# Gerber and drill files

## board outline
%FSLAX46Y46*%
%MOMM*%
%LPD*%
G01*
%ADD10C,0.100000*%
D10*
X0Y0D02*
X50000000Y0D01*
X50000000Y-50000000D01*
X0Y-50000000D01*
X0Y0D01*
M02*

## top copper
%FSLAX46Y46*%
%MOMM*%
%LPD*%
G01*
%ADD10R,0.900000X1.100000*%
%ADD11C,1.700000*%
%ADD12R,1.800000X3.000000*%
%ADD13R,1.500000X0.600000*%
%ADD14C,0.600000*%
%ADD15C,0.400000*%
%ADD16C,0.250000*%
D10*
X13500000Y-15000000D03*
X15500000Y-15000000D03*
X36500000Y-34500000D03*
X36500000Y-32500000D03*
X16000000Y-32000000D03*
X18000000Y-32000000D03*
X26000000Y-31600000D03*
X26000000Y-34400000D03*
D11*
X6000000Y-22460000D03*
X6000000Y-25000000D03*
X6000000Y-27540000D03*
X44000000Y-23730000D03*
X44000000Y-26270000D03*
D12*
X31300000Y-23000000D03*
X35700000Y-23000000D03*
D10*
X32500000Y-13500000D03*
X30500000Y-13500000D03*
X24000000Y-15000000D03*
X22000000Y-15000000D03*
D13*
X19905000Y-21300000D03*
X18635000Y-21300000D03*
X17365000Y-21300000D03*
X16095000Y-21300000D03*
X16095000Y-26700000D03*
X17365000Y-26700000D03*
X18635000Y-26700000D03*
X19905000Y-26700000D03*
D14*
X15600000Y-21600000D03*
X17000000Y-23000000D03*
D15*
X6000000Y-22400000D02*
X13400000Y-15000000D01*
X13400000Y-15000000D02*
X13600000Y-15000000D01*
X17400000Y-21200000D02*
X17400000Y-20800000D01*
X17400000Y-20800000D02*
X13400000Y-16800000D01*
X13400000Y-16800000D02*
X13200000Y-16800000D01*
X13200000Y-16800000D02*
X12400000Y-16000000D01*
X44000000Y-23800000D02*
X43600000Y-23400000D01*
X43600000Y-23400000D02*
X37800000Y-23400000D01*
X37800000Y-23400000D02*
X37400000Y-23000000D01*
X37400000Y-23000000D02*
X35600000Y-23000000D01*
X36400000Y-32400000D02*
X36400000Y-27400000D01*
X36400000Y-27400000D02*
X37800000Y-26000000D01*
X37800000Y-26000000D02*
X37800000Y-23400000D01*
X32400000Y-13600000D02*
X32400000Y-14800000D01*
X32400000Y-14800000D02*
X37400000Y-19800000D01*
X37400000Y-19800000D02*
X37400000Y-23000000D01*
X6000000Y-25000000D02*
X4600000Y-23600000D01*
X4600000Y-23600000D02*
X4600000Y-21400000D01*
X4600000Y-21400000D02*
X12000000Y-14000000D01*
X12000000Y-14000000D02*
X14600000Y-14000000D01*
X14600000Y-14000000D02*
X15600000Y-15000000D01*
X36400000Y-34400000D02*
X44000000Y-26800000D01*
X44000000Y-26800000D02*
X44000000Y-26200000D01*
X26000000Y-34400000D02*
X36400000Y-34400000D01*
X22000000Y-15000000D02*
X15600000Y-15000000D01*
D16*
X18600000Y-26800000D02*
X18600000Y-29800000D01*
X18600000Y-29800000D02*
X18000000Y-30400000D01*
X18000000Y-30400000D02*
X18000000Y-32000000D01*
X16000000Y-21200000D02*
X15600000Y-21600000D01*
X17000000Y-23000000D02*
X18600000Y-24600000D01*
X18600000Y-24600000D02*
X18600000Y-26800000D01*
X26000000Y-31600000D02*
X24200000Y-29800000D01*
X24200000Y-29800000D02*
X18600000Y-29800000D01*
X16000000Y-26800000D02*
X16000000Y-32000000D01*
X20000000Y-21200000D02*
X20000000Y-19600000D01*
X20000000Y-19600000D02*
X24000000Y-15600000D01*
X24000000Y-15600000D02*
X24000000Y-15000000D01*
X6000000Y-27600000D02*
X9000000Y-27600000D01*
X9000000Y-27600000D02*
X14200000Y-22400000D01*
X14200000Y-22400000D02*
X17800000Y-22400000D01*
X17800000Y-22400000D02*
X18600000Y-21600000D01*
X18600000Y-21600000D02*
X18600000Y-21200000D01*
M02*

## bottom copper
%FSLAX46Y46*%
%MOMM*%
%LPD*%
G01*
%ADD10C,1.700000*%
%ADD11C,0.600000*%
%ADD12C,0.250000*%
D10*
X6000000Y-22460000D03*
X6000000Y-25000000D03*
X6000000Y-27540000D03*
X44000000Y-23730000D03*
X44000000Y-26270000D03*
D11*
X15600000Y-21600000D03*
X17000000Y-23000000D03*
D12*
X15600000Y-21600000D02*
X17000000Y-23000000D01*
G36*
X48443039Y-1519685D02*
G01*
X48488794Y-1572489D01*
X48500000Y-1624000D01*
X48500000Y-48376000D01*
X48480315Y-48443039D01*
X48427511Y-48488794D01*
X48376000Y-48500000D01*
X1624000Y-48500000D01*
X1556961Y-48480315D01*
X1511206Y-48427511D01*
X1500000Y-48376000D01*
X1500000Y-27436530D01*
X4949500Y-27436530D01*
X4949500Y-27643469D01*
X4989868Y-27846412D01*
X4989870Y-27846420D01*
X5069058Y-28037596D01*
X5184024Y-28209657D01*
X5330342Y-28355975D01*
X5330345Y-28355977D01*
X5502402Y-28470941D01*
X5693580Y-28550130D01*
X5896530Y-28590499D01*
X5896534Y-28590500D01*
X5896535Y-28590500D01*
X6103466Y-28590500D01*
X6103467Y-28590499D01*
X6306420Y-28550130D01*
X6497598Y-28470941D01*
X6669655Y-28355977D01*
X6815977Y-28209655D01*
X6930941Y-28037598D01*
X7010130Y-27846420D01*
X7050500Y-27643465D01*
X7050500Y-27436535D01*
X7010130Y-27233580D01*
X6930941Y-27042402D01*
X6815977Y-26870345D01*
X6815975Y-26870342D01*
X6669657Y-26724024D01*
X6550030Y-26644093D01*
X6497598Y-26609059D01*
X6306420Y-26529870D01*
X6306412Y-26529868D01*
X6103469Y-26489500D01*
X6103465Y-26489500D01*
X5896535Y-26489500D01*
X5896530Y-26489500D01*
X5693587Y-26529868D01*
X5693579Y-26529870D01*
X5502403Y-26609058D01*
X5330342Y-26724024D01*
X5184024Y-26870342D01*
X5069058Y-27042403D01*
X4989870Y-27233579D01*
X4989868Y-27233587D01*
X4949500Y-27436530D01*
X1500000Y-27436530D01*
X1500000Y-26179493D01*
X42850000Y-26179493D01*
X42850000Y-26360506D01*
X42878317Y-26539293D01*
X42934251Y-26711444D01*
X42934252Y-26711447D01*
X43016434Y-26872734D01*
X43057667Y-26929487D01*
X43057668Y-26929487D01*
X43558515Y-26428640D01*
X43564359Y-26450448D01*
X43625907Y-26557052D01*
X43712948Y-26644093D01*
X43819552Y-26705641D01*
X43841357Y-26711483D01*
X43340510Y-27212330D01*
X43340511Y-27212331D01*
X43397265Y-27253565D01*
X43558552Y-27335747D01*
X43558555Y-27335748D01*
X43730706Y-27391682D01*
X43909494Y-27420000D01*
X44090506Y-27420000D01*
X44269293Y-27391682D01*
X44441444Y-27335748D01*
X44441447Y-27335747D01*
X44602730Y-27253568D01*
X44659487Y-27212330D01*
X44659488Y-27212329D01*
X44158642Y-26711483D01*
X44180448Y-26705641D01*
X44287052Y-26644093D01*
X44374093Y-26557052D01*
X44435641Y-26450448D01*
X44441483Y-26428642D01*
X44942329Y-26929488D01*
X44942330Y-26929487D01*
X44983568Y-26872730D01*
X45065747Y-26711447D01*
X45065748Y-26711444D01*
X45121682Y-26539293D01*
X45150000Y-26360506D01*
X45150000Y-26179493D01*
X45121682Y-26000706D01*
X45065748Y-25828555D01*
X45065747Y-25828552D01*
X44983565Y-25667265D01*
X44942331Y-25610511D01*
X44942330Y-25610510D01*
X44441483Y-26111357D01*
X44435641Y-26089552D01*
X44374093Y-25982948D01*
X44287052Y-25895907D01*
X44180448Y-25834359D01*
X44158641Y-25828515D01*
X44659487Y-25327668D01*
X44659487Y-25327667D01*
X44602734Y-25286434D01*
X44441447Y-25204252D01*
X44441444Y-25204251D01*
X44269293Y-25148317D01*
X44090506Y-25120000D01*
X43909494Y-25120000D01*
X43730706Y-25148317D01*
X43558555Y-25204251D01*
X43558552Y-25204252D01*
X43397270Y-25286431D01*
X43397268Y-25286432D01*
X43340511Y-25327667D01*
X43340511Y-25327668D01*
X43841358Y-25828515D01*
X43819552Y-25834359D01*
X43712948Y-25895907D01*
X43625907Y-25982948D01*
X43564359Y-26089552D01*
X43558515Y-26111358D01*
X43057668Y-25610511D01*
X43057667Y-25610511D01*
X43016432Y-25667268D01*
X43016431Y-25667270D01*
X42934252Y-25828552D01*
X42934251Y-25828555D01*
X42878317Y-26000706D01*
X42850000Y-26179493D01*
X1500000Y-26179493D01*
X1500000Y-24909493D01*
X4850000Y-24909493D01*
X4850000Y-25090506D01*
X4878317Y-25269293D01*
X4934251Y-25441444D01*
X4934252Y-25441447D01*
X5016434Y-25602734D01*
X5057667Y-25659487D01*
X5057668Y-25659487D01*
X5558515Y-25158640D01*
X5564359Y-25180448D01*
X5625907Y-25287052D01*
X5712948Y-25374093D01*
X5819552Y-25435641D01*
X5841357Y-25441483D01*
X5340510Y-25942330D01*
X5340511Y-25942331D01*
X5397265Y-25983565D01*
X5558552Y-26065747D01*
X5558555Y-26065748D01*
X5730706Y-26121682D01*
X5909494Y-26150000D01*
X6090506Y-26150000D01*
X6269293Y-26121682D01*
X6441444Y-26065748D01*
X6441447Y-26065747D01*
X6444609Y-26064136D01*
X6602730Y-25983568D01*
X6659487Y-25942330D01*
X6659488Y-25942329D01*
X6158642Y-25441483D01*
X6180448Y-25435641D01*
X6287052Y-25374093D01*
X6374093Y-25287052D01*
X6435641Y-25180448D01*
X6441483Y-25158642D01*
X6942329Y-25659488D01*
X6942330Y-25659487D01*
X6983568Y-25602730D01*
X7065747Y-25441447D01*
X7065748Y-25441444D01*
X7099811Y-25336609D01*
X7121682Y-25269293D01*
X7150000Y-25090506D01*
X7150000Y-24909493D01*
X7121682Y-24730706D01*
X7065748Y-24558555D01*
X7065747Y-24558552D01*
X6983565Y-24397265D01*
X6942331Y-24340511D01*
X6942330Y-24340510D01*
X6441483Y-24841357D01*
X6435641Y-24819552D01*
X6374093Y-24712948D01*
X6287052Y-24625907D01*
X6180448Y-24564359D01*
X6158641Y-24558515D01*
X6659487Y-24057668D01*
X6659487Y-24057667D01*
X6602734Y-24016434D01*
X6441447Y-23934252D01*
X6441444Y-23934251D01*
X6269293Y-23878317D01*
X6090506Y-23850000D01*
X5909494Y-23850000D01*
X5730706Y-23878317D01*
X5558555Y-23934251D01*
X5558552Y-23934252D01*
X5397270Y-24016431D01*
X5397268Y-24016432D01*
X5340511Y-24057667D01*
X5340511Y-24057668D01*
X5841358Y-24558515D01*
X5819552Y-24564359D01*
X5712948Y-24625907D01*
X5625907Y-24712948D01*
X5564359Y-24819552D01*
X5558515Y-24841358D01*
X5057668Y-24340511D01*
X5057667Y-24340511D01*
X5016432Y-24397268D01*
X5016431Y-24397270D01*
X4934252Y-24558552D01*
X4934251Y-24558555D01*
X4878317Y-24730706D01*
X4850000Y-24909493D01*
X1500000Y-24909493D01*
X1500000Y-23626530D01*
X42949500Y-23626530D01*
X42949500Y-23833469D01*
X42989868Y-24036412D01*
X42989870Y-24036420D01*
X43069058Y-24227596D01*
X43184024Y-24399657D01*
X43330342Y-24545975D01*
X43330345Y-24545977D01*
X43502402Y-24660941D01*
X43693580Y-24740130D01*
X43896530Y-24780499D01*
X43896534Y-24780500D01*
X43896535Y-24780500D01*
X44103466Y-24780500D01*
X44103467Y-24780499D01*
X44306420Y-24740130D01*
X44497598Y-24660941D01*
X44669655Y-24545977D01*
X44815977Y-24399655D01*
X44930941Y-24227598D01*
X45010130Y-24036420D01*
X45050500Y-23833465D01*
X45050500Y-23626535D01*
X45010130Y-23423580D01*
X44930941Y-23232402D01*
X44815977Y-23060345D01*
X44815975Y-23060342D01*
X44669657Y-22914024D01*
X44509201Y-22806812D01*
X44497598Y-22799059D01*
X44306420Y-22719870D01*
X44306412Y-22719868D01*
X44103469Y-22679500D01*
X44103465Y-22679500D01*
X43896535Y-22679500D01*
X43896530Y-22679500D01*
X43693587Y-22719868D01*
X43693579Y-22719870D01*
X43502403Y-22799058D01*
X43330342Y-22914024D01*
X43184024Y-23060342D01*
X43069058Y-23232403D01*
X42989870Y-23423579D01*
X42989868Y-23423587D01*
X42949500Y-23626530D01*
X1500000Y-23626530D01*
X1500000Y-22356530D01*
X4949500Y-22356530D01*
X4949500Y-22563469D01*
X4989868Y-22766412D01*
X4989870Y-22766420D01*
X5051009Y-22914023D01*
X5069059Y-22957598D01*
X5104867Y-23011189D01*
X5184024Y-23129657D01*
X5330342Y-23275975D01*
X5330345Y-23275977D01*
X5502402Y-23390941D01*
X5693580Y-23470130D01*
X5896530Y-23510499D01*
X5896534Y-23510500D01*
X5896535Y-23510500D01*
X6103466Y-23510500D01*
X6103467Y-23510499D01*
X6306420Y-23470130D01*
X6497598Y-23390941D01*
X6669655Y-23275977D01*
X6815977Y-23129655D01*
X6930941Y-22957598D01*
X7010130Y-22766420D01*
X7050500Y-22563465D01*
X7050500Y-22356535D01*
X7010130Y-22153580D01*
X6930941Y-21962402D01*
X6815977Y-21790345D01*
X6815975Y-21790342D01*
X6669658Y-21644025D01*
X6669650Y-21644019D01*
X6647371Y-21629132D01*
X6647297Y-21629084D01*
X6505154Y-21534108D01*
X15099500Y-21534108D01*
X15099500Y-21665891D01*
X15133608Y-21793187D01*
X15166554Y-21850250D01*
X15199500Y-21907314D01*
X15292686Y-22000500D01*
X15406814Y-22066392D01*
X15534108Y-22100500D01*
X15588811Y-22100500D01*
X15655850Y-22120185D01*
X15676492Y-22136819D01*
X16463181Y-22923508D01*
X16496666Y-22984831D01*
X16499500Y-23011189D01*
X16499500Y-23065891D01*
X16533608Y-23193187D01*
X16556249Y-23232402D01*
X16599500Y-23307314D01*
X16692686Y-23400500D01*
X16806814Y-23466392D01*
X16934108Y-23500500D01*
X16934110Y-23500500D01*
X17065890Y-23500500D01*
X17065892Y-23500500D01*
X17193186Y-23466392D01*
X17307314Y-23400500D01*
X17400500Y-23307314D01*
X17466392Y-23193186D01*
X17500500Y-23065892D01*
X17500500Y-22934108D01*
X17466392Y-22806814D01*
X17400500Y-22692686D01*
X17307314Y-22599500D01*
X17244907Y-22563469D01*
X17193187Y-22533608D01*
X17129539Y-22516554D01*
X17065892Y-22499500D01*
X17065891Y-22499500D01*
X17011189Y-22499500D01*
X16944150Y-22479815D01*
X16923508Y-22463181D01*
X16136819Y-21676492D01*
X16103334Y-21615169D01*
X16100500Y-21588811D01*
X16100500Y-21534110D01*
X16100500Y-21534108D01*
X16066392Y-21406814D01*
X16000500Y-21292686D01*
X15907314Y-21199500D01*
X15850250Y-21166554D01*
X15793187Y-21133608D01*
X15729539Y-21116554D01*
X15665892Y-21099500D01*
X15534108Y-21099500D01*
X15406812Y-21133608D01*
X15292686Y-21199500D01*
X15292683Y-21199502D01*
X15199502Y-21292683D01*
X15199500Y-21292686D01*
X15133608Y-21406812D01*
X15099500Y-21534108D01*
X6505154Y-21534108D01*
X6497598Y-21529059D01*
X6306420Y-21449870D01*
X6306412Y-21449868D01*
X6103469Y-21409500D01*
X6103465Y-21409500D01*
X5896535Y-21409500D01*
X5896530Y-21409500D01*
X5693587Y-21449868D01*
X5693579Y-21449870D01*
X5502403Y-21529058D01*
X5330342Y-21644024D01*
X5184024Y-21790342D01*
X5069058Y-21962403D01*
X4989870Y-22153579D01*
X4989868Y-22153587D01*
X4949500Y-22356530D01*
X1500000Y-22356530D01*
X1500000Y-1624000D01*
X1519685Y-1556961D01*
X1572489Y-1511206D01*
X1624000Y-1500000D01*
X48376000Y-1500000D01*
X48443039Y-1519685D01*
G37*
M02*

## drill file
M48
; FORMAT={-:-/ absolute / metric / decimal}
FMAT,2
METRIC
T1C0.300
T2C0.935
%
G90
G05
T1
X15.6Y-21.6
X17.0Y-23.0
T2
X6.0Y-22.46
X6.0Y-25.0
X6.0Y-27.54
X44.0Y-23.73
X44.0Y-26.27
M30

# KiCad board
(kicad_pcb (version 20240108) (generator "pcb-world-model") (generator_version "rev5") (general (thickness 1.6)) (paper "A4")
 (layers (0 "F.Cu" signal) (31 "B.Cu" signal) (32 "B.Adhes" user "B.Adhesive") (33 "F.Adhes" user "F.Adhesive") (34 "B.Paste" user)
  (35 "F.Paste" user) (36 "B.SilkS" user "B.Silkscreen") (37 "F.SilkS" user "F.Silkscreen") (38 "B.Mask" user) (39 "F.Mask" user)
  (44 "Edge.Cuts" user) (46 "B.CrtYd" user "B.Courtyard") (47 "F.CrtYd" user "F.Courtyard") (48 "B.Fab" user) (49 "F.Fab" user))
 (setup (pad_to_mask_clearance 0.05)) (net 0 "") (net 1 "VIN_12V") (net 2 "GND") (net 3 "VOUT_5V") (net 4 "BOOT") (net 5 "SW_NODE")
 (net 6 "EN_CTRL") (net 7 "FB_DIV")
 (gr_rect (start 0.0 0.0) (end 50.0000 50.0000) (stroke (width 0.1) (type default)) (fill none) (layer "Edge.Cuts"))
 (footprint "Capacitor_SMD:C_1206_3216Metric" (layer "F.Cu") (at 14.5000 15.0000 0)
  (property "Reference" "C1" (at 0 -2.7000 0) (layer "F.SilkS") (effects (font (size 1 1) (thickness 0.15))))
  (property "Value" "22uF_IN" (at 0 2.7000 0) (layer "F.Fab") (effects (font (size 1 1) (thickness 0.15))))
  (pad "1" smd rect (at -1.0000 0.0000) (size 0.9000 1.1000) (layers "F.Cu" "F.Paste" "F.Mask") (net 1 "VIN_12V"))
  (pad "2" smd rect (at 1.0000 0.0000) (size 0.9000 1.1000) (layers "F.Cu" "F.Paste" "F.Mask") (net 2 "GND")))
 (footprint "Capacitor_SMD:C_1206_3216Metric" (layer "F.Cu") (at 36.5000 33.5000 90)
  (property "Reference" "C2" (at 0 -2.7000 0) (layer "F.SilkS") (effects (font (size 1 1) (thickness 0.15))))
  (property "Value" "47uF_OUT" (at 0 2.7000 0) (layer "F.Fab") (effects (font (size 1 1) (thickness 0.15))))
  (pad "1" smd rect (at -1.0000 0.0000) (size 0.9000 1.1000) (layers "F.Cu" "F.Paste" "F.Mask") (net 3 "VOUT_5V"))
  (pad "2" smd rect (at 1.0000 0.0000) (size 0.9000 1.1000) (layers "F.Cu" "F.Paste" "F.Mask") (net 2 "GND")))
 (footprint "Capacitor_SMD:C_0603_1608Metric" (layer "F.Cu") (at 17.0000 32.0000 0)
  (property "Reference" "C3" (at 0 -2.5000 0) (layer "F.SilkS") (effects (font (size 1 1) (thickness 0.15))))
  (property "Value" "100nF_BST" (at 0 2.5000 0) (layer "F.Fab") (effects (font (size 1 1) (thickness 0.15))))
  (pad "1" smd rect (at -1.0000 0.0000) (size 0.9000 1.1000) (layers "F.Cu" "F.Paste" "F.Mask") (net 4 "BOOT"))
  (pad "2" smd rect (at 1.0000 0.0000) (size 0.9000 1.1000) (layers "F.Cu" "F.Paste" "F.Mask") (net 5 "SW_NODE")))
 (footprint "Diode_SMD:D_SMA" (layer "F.Cu") (at 26.0000 33.0000 270)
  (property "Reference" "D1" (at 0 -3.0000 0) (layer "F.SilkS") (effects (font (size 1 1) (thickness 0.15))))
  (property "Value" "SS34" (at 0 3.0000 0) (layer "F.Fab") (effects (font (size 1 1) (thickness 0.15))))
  (pad "1" smd rect (at -1.4000 0.0000) (size 0.9000 1.1000) (layers "F.Cu" "F.Paste" "F.Mask") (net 2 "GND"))
  (pad "2" smd rect (at 1.4000 0.0000) (size 0.9000 1.1000) (layers "F.Cu" "F.Paste" "F.Mask") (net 5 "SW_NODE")))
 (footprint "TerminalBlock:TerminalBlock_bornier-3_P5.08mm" (layer "F.Cu") (at 6.0000 25.0000 0) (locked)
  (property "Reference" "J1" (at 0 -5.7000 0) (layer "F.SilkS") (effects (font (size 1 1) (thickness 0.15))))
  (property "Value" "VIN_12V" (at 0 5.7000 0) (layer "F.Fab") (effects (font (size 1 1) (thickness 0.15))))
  (pad "1" thru_hole circle (at 0.0000 -2.5400) (size 1.7000 1.7000) (drill 0.9350) (layers "*.Cu" "*.Mask") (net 1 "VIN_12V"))
  (pad "2" thru_hole circle (at 0.0000 0.0000) (size 1.7000 1.7000) (drill 0.9350) (layers "*.Cu" "*.Mask") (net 2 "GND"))
  (pad "3" thru_hole circle (at 0.0000 2.5400) (size 1.7000 1.7000) (drill 0.9350) (layers "*.Cu" "*.Mask") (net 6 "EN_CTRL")))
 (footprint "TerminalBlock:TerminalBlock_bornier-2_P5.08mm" (layer "F.Cu") (at 44.0000 25.0000 0) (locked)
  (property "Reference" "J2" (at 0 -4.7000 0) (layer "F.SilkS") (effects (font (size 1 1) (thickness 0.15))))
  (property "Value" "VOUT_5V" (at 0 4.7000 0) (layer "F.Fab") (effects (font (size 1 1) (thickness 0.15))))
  (pad "1" thru_hole circle (at 0.0000 -1.2700) (size 1.7000 1.7000) (drill 0.9350) (layers "*.Cu" "*.Mask") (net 3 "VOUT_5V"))
  (pad "2" thru_hole circle (at 0.0000 1.2700) (size 1.7000 1.7000) (drill 0.9350) (layers "*.Cu" "*.Mask") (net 2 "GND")))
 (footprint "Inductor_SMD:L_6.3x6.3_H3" (layer "F.Cu") (at 33.5000 23.0000 0)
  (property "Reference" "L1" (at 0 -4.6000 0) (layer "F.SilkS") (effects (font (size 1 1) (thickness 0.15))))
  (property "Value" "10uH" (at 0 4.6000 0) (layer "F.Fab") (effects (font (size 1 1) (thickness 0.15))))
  (pad "1" smd rect (at -2.2000 0.0000) (size 1.8000 3.0000) (layers "F.Cu" "F.Paste" "F.Mask") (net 5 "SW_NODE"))
  (pad "2" smd rect (at 2.2000 0.0000) (size 1.8000 3.0000) (layers "F.Cu" "F.Paste" "F.Mask") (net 3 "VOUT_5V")))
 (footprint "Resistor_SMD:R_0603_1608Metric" (layer "F.Cu") (at 31.5000 13.5000 180)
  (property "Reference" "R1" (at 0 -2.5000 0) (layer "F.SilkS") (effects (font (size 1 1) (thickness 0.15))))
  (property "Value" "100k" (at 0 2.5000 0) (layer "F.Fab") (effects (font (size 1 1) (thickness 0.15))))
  (pad "1" smd rect (at -1.0000 0.0000) (size 0.9000 1.1000) (layers "F.Cu" "F.Paste" "F.Mask") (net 3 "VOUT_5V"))
  (pad "2" smd rect (at 1.0000 0.0000) (size 0.9000 1.1000) (layers "F.Cu" "F.Paste" "F.Mask") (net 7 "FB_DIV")))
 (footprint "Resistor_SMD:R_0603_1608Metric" (layer "F.Cu") (at 23.0000 15.0000 180)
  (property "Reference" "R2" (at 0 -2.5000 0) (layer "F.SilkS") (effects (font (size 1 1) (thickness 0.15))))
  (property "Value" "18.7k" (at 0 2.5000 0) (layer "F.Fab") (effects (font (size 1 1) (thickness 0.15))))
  (pad "1" smd rect (at -1.0000 0.0000) (size 0.9000 1.1000) (layers "F.Cu" "F.Paste" "F.Mask") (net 7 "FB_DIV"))
  (pad "2" smd rect (at 1.0000 0.0000) (size 0.9000 1.1000) (layers "F.Cu" "F.Paste" "F.Mask") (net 2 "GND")))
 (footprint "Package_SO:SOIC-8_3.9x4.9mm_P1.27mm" (layer "F.Cu") (at 18.0000 24.0000 270)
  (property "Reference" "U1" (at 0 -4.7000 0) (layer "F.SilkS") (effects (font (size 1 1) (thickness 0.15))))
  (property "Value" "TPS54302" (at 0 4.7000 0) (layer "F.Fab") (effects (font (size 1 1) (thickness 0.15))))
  (pad "1" smd rect (at -2.7000 -1.9050) (size 1.5000 0.6000) (layers "F.Cu" "F.Paste" "F.Mask") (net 4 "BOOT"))
  (pad "2" smd rect (at -2.7000 -0.6350) (size 1.5000 0.6000) (layers "F.Cu" "F.Paste" "F.Mask") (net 1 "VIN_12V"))
  (pad "3" smd rect (at -2.7000 0.6350) (size 1.5000 0.6000) (layers "F.Cu" "F.Paste" "F.Mask") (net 5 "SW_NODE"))
  (pad "4" smd rect (at -2.7000 1.9050) (size 1.5000 0.6000) (layers "F.Cu" "F.Paste" "F.Mask") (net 2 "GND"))
  (pad "5" smd rect (at 2.7000 1.9050) (size 1.5000 0.6000) (layers "F.Cu" "F.Paste" "F.Mask") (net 7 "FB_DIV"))
  (pad "6" smd rect (at 2.7000 0.6350) (size 1.5000 0.6000) (layers "F.Cu" "F.Paste" "F.Mask") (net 6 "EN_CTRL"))
  (pad "7" smd rect (at 2.7000 -0.6350) (size 1.5000 0.6000) (layers "F.Cu" "F.Paste" "F.Mask") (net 1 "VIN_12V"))
  (pad "8" smd rect (at 2.7000 -1.9050) (size 1.5000 0.6000) (layers "F.Cu" "F.Paste" "F.Mask") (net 5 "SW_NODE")))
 (segment (start 6.0000 22.4000) (end 13.4000 15.0000) (width 0.4000) (layer "F.Cu") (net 1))
 (segment (start 13.4000 15.0000) (end 13.6000 15.0000) (width 0.4000) (layer "F.Cu") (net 1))
 (segment (start 17.4000 21.2000) (end 17.4000 20.8000) (width 0.4000) (layer "F.Cu") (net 1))
 (segment (start 17.4000 20.8000) (end 13.4000 16.8000) (width 0.4000) (layer "F.Cu") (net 1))
 (segment (start 13.4000 16.8000) (end 13.2000 16.8000) (width 0.4000) (layer "F.Cu") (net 1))
 (segment (start 13.2000 16.8000) (end 12.4000 16.0000) (width 0.4000) (layer "F.Cu") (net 1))
 (segment (start 44.0000 23.8000) (end 43.6000 23.4000) (width 0.4000) (layer "F.Cu") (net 3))
 (segment (start 43.6000 23.4000) (end 37.8000 23.4000) (width 0.4000) (layer "F.Cu") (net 3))
 (segment (start 37.8000 23.4000) (end 37.4000 23.0000) (width 0.4000) (layer "F.Cu") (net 3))
 (segment (start 37.4000 23.0000) (end 35.6000 23.0000) (width 0.4000) (layer "F.Cu") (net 3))
 (segment (start 36.4000 32.4000) (end 36.4000 27.4000) (width 0.4000) (layer "F.Cu") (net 3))
 (segment (start 36.4000 27.4000) (end 37.8000 26.0000) (width 0.4000) (layer "F.Cu") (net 3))
 (segment (start 37.8000 26.0000) (end 37.8000 23.4000) (width 0.4000) (layer "F.Cu") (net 3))
 (segment (start 32.4000 13.6000) (end 32.4000 14.8000) (width 0.4000) (layer "F.Cu") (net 3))
 (segment (start 32.4000 14.8000) (end 37.4000 19.8000) (width 0.4000) (layer "F.Cu") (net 3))
 (segment (start 37.4000 19.8000) (end 37.4000 23.0000) (width 0.4000) (layer "F.Cu") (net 3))
 (segment (start 6.0000 25.0000) (end 4.6000 23.6000) (width 0.4000) (layer "F.Cu") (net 2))
 (segment (start 4.6000 23.6000) (end 4.6000 21.4000) (width 0.4000) (layer "F.Cu") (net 2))
 (segment (start 4.6000 21.4000) (end 12.0000 14.0000) (width 0.4000) (layer "F.Cu") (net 2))
 (segment (start 12.0000 14.0000) (end 14.6000 14.0000) (width 0.4000) (layer "F.Cu") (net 2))
 (segment (start 14.6000 14.0000) (end 15.6000 15.0000) (width 0.4000) (layer "F.Cu") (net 2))
 (segment (start 36.4000 34.4000) (end 44.0000 26.8000) (width 0.4000) (layer "F.Cu") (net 2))
 (segment (start 44.0000 26.8000) (end 44.0000 26.2000) (width 0.4000) (layer "F.Cu") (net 2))
 (segment (start 26.0000 34.4000) (end 36.4000 34.4000) (width 0.4000) (layer "F.Cu") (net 2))
 (segment (start 22.0000 15.0000) (end 15.6000 15.0000) (width 0.4000) (layer "F.Cu") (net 2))
 (segment (start 18.6000 26.8000) (end 18.6000 29.8000) (width 0.2500) (layer "F.Cu") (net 5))
 (segment (start 18.6000 29.8000) (end 18.0000 30.4000) (width 0.2500) (layer "F.Cu") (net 5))
 (segment (start 18.0000 30.4000) (end 18.0000 32.0000) (width 0.2500) (layer "F.Cu") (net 5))
 (segment (start 16.0000 21.2000) (end 15.6000 21.6000) (width 0.2500) (layer "F.Cu") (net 5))
 (segment (start 15.6000 21.6000) (end 17.0000 23.0000) (width 0.2500) (layer "B.Cu") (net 5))
 (segment (start 17.0000 23.0000) (end 18.6000 24.6000) (width 0.2500) (layer "F.Cu") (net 5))
 (segment (start 18.6000 24.6000) (end 18.6000 26.8000) (width 0.2500) (layer "F.Cu") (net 5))
 (segment (start 26.0000 31.6000) (end 24.2000 29.8000) (width 0.2500) (layer "F.Cu") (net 5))
 (segment (start 24.2000 29.8000) (end 18.6000 29.8000) (width 0.2500) (layer "F.Cu") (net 5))
 (segment (start 16.0000 26.8000) (end 16.0000 32.0000) (width 0.2500) (layer "F.Cu") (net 4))
 (segment (start 20.0000 21.2000) (end 20.0000 19.6000) (width 0.2500) (layer "F.Cu") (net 7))
 (segment (start 20.0000 19.6000) (end 24.0000 15.6000) (width 0.2500) (layer "F.Cu") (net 7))
 (segment (start 24.0000 15.6000) (end 24.0000 15.0000) (width 0.2500) (layer "F.Cu") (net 7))
 (segment (start 6.0000 27.6000) (end 9.0000 27.6000) (width 0.2500) (layer "F.Cu") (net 6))
 (segment (start 9.0000 27.6000) (end 14.2000 22.4000) (width 0.2500) (layer "F.Cu") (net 6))
 (segment (start 14.2000 22.4000) (end 17.8000 22.4000) (width 0.2500) (layer "F.Cu") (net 6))
 (segment (start 17.8000 22.4000) (end 18.6000 21.6000) (width 0.2500) (layer "F.Cu") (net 6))
 (segment (start 18.6000 21.6000) (end 18.6000 21.2000) (width 0.2500) (layer "F.Cu") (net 6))
 (via (at 15.6000 21.6000) (size 0.6000) (drill 0.3000) (layers "F.Cu" "B.Cu") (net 5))
 (via (at 17.0000 23.0000) (size 0.6000) (drill 0.3000) (layers "F.Cu" "B.Cu") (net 5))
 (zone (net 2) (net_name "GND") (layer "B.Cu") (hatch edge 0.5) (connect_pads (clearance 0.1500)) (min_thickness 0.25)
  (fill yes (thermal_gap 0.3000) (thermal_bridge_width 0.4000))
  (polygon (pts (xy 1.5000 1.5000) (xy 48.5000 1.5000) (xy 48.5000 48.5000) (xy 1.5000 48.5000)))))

